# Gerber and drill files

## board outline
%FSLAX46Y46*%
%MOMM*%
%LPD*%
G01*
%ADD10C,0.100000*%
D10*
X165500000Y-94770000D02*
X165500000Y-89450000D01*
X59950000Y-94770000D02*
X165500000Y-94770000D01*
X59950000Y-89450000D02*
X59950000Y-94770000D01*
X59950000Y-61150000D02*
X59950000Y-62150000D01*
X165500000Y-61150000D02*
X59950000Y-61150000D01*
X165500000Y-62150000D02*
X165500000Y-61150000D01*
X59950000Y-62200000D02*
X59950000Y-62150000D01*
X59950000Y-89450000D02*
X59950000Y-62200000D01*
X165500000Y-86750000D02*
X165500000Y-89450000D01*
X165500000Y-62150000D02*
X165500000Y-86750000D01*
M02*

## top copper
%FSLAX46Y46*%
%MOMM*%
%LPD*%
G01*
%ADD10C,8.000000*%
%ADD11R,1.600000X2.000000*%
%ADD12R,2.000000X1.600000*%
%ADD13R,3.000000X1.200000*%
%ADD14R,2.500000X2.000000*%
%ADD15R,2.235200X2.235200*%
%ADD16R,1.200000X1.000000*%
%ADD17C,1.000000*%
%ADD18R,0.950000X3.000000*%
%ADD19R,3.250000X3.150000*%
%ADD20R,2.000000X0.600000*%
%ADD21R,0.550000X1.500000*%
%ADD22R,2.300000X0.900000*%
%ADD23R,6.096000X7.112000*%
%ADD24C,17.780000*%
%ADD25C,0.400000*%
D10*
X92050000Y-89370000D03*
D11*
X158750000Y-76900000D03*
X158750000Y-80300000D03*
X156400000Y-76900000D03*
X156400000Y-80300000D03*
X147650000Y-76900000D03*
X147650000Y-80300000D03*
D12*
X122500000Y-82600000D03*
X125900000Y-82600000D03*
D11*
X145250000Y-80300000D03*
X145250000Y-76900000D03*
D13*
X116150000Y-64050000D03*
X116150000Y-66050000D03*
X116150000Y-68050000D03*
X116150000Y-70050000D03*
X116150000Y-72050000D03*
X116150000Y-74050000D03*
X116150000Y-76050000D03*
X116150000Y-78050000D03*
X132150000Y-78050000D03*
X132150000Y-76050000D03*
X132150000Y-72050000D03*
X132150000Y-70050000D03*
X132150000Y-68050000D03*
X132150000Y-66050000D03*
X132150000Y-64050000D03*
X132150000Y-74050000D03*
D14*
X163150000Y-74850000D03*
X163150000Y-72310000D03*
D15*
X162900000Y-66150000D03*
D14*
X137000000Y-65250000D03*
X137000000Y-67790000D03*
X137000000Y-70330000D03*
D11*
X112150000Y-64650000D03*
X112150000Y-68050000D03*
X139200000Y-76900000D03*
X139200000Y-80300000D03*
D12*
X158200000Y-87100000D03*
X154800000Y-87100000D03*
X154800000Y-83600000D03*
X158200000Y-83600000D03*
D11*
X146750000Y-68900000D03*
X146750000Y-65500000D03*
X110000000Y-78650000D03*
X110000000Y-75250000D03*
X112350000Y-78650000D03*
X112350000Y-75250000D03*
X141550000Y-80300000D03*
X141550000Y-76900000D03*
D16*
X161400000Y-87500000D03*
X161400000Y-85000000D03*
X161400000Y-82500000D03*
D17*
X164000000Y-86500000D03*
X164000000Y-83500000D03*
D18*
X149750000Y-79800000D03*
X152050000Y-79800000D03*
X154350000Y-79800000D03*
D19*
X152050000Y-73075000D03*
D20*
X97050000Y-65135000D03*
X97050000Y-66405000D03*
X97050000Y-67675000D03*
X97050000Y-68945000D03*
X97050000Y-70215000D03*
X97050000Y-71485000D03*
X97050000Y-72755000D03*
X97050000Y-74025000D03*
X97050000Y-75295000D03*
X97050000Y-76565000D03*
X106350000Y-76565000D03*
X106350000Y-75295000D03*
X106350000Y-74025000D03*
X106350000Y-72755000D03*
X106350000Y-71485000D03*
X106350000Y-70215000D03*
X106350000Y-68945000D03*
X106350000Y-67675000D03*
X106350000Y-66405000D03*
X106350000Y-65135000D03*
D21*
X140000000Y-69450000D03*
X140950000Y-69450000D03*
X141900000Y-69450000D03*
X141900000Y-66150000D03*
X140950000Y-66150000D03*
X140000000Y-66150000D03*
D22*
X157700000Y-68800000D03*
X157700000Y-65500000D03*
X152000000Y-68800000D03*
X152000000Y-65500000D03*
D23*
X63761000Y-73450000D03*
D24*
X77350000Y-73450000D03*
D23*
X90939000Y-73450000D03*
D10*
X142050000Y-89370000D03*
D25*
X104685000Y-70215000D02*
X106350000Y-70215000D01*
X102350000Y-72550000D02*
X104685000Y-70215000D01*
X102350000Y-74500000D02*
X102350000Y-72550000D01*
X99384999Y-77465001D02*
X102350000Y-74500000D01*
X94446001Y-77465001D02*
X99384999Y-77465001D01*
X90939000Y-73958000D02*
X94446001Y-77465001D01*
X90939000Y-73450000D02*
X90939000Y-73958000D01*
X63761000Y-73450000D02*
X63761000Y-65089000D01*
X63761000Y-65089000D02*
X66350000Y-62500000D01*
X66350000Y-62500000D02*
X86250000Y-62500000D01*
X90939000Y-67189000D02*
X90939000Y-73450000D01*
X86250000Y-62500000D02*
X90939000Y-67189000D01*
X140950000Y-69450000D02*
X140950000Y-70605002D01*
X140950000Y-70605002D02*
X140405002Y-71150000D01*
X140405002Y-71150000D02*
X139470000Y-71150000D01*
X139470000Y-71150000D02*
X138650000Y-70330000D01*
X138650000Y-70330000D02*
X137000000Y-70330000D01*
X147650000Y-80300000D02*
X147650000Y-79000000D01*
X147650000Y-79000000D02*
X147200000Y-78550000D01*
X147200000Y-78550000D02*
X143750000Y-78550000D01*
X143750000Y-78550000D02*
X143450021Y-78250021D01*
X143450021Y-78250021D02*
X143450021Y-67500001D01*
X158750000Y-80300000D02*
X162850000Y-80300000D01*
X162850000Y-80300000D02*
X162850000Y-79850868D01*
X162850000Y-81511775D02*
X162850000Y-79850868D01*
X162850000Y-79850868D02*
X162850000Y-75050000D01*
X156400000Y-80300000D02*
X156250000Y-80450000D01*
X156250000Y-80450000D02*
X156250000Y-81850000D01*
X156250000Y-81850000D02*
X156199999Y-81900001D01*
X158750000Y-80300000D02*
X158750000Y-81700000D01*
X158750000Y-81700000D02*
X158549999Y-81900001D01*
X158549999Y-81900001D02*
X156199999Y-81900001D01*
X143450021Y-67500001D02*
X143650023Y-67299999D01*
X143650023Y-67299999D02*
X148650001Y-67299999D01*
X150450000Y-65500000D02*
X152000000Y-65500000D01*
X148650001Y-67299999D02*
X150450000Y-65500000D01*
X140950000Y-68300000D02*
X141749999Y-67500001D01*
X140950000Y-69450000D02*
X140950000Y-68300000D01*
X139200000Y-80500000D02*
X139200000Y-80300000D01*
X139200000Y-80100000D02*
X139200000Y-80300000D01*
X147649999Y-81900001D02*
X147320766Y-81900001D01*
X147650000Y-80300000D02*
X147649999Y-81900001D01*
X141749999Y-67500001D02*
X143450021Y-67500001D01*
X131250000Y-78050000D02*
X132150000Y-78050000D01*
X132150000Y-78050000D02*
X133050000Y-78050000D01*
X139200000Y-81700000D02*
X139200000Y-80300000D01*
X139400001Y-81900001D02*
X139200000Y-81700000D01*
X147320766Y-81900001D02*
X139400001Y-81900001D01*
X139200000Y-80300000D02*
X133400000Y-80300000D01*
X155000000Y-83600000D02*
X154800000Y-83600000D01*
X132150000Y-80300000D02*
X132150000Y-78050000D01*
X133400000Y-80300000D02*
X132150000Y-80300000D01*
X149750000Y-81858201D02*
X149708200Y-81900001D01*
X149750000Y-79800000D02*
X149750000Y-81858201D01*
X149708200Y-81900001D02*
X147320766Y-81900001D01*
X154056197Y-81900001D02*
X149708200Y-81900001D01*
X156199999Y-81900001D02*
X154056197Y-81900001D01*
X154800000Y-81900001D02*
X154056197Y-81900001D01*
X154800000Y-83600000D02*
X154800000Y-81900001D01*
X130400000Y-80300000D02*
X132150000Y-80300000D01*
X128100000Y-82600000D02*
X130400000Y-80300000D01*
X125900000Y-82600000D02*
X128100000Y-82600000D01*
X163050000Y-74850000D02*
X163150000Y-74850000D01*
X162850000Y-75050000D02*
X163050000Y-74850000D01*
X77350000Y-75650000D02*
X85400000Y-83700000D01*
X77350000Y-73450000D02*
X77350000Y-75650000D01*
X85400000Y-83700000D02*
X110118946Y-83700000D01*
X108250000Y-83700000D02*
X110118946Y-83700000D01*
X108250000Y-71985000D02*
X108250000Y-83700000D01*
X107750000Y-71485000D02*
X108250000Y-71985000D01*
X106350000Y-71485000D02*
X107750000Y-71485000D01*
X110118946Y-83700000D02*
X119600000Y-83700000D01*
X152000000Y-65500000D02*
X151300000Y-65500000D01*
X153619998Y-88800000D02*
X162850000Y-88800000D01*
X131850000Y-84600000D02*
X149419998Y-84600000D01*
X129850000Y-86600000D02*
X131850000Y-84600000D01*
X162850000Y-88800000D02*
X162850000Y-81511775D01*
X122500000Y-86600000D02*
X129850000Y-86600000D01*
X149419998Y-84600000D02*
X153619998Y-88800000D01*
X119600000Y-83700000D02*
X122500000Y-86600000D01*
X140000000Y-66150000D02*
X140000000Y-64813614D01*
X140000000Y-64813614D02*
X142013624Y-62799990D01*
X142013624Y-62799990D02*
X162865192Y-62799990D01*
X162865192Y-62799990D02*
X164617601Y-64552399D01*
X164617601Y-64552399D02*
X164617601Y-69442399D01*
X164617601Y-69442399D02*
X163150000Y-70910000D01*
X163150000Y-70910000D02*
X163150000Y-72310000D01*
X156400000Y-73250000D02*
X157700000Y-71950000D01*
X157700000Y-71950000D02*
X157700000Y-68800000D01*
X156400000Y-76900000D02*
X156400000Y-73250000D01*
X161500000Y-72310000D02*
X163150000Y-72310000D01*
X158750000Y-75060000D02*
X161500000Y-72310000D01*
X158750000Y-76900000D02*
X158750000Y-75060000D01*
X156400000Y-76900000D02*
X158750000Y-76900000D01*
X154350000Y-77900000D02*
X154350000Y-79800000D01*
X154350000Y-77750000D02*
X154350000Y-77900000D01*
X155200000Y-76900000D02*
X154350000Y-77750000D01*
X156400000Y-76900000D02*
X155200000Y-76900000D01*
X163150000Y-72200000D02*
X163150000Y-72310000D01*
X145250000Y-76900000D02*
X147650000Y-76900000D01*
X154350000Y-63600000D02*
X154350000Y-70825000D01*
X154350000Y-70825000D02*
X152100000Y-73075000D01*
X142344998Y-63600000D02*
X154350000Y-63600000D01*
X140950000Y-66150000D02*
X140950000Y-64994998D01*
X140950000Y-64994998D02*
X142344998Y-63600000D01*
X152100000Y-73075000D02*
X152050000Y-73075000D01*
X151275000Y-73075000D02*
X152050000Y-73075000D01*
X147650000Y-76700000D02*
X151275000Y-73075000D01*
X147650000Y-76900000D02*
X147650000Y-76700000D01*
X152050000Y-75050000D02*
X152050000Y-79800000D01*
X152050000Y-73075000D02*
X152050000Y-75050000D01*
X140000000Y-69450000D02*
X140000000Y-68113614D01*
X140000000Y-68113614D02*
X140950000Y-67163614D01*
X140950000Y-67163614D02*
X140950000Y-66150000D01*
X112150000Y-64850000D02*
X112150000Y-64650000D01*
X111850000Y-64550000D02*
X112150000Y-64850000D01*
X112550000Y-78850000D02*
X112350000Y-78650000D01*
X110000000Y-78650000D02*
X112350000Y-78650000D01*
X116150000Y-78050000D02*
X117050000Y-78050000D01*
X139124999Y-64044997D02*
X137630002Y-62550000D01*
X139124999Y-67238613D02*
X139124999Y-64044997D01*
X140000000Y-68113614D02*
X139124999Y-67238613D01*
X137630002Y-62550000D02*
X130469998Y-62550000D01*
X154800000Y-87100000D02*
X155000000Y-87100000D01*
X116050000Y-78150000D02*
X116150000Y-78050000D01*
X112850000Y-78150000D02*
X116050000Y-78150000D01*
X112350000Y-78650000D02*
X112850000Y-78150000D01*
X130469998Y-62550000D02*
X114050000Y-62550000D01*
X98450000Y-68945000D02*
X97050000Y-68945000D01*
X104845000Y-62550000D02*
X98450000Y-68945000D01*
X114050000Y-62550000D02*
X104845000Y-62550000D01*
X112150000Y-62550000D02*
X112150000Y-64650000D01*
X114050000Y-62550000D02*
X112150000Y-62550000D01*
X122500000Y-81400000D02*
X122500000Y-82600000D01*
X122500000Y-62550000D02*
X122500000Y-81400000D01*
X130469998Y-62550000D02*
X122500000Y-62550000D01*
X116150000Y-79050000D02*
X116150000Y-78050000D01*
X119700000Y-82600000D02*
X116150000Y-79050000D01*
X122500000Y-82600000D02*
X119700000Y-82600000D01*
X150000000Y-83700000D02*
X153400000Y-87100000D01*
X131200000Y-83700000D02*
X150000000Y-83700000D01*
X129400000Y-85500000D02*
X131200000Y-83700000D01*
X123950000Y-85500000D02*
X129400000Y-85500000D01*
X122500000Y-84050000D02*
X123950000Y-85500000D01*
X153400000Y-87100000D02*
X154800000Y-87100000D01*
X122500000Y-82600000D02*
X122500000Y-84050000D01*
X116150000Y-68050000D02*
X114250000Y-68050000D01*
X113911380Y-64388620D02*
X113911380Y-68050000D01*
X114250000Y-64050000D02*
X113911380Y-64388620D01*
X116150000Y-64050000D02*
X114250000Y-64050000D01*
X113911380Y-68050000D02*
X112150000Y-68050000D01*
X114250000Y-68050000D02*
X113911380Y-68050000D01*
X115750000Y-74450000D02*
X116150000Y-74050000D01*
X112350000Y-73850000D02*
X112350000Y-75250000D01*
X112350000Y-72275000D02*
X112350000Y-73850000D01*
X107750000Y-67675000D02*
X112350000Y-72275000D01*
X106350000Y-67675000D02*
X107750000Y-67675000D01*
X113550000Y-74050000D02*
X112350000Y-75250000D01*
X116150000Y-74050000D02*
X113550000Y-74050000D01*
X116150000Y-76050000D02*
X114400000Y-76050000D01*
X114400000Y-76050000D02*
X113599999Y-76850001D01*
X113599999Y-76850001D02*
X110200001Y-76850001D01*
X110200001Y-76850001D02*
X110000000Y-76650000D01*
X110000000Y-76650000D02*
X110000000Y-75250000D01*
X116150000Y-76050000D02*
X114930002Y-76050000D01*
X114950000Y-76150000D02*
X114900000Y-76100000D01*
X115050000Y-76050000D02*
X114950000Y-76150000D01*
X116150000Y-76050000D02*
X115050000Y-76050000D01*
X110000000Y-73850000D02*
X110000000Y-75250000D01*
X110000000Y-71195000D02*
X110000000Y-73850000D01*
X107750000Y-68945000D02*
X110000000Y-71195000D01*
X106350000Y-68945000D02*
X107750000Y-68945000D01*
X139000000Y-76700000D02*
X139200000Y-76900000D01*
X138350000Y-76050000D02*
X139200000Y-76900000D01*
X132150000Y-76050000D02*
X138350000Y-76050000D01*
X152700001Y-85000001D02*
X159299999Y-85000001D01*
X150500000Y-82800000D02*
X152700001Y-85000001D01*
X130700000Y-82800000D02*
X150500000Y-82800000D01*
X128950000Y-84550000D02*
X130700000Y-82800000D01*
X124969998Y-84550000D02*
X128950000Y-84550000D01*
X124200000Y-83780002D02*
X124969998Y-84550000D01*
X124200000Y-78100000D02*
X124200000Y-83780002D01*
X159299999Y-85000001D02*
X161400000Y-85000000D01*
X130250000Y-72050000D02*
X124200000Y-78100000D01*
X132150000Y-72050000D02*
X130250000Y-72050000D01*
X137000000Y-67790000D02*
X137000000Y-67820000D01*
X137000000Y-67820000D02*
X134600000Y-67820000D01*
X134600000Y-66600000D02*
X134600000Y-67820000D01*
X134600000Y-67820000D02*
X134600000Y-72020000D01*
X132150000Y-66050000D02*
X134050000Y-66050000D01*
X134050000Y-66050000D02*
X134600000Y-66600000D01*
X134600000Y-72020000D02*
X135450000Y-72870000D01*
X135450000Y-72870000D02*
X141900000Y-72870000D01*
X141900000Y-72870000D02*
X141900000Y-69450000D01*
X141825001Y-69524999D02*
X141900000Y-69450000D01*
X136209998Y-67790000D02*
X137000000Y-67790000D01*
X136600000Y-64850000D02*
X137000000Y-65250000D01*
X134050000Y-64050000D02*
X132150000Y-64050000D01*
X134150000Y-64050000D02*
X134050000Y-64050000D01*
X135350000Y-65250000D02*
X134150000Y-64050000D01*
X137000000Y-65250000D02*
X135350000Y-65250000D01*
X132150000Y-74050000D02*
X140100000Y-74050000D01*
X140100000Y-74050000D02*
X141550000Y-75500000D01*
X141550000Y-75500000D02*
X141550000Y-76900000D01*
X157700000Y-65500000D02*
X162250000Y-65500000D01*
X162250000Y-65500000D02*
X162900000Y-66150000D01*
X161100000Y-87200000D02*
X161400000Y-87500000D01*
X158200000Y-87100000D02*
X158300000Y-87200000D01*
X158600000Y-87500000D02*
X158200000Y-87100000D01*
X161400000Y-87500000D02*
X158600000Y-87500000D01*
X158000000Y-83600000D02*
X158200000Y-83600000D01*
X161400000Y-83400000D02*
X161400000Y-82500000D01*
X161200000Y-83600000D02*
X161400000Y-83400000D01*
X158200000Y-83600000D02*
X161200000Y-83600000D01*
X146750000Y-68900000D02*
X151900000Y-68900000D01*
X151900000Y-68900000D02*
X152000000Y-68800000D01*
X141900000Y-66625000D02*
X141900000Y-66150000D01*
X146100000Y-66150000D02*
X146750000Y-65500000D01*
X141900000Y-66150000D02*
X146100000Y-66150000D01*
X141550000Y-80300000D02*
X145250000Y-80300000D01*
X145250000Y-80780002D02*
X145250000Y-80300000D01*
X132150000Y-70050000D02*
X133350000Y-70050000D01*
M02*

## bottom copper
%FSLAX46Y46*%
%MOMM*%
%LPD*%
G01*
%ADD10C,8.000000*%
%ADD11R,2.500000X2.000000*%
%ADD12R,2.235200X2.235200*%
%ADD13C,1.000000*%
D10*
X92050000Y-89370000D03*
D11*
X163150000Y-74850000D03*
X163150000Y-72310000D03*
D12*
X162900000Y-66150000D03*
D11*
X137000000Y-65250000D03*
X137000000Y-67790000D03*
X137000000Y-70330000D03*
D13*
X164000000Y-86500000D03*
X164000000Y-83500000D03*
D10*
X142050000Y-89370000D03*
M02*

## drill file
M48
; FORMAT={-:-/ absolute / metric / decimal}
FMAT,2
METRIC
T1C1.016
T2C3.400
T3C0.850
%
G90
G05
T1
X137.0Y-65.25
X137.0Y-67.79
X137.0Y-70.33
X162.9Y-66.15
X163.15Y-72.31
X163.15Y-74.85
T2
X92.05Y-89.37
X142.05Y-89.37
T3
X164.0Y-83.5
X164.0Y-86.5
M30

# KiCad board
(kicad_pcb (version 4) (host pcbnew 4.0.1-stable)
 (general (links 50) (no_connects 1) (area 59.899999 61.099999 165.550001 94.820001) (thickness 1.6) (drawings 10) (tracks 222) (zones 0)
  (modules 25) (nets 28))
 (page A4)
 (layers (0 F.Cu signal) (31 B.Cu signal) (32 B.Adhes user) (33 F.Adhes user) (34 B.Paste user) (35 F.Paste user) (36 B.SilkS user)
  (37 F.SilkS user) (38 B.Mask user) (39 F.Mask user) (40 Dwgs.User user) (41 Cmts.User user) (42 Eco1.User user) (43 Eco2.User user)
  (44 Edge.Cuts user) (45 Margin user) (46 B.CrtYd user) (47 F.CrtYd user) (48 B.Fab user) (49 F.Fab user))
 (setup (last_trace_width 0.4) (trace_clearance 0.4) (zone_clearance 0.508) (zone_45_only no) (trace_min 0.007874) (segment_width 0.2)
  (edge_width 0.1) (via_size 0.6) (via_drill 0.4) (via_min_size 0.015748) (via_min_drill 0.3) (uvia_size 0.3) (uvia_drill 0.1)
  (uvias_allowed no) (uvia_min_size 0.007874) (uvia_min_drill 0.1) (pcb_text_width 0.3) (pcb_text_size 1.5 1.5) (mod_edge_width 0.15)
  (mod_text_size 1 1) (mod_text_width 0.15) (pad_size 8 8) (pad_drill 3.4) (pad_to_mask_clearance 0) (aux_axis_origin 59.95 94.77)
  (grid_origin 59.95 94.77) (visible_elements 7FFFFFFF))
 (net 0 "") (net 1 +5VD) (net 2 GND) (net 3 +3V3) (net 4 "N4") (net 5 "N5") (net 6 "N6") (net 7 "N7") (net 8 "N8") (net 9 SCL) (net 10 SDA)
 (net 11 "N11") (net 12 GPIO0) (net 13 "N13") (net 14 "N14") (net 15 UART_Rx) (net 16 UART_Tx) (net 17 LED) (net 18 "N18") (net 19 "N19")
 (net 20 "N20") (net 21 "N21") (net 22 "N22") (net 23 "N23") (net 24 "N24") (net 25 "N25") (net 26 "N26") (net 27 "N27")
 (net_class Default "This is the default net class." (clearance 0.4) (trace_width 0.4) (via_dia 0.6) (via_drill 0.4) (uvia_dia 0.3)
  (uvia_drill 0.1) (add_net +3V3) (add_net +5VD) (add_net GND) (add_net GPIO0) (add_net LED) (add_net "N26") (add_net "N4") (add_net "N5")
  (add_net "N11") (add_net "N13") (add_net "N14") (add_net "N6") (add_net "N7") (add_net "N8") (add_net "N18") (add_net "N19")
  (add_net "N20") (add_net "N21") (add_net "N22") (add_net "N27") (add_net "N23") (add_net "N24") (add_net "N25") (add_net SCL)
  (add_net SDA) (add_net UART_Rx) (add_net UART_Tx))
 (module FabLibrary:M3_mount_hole (layer F.Cu) (at 92.05 89.37)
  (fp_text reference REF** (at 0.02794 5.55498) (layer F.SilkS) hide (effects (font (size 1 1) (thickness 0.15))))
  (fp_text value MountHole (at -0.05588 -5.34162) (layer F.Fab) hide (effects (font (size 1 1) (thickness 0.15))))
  (pad 1 thru_hole circle (at 0 0) (size 8 8) (drill 3.4) (layers *.Cu *.Mask F.SilkS)))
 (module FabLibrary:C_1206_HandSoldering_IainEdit (layer F.Cu) (at 158.75 78.6 270)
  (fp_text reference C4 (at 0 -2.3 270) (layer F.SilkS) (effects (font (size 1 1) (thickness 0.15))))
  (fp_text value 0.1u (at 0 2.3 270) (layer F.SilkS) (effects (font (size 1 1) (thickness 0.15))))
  (pad 1 smd rect (at -1.7 0 270) (size 2 1.6) (layers F.Cu F.Paste F.Mask) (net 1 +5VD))
  (pad 2 smd rect (at 1.7 0 270) (size 2 1.6) (layers F.Cu F.Paste F.Mask) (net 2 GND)))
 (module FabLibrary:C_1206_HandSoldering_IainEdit (layer F.Cu) (at 156.4 78.6 270)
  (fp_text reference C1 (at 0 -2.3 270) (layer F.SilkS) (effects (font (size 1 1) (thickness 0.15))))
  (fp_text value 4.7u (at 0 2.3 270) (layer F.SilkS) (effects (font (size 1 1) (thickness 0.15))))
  (pad 1 smd rect (at -1.7 0 270) (size 2 1.6) (layers F.Cu F.Paste F.Mask) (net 1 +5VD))
  (pad 2 smd rect (at 1.7 0 270) (size 2 1.6) (layers F.Cu F.Paste F.Mask) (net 2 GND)))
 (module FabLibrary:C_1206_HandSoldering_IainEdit (layer F.Cu) (at 147.65 78.6 270)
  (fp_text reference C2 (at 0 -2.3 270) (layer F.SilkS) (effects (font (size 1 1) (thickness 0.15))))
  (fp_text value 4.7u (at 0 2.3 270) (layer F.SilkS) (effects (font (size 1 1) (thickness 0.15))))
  (pad 1 smd rect (at -1.7 0 270) (size 2 1.6) (layers F.Cu F.Paste F.Mask) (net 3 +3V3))
  (pad 2 smd rect (at 1.7 0 270) (size 2 1.6) (layers F.Cu F.Paste F.Mask) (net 2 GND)))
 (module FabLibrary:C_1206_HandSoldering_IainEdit (layer F.Cu) (at 124.2 82.6)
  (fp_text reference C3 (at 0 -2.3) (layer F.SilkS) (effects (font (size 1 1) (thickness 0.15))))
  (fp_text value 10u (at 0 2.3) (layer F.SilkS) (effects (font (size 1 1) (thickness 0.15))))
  (pad 1 smd rect (at -1.7 0) (size 2 1.6) (layers F.Cu F.Paste F.Mask) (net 3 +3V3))
  (pad 2 smd rect (at 1.7 0) (size 2 1.6) (layers F.Cu F.Paste F.Mask) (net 2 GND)))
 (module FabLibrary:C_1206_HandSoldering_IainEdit (layer F.Cu) (at 145.25 78.6 90)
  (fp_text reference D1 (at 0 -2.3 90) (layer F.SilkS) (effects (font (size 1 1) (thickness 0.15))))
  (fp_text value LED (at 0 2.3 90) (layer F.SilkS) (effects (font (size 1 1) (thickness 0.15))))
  (pad 1 smd rect (at -1.7 0 90) (size 2 1.6) (layers F.Cu F.Paste F.Mask) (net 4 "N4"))
  (pad 2 smd rect (at 1.7 0 90) (size 2 1.6) (layers F.Cu F.Paste F.Mask) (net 3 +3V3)))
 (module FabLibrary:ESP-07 (layer F.Cu) (at 124.15 70.05 270)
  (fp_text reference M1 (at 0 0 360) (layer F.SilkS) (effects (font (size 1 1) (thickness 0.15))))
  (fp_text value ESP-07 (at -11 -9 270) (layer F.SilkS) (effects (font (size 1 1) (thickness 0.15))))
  (pad 1 smd rect (at -6 8 270) (size 1.2 3) (layers F.Cu F.Paste F.Mask) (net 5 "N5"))
  (pad 2 smd rect (at -4 8 270) (size 1.2 3) (layers F.Cu F.Paste F.Mask) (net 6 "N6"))
  (pad 3 smd rect (at -2 8 270) (size 1.2 3) (layers F.Cu F.Paste F.Mask) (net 5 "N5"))
  (pad 4 smd rect (at 0 8 270) (size 1.2 3) (layers F.Cu F.Paste F.Mask) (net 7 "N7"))
  (pad 5 smd rect (at 2 8 270) (size 1.2 3) (layers F.Cu F.Paste F.Mask) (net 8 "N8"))
  (pad 6 smd rect (at 4 8 270) (size 1.2 3) (layers F.Cu F.Paste F.Mask) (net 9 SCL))
  (pad 7 smd rect (at 6 8 270) (size 1.2 3) (layers F.Cu F.Paste F.Mask) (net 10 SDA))
  (pad 8 smd rect (at 8 8 270) (size 1.2 3) (layers F.Cu F.Paste F.Mask) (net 3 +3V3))
  (pad 9 smd rect (at 8 -8 270) (size 1.2 3) (layers F.Cu F.Paste F.Mask) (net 2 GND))
  (pad 10 smd rect (at 6 -8 270) (size 1.2 3) (layers F.Cu F.Paste F.Mask) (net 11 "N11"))
  (pad 12 smd rect (at 2 -8 270) (size 1.2 3) (layers F.Cu F.Paste F.Mask) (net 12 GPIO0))
  (pad 13 smd rect (at 0 -8 270) (size 1.2 3) (layers F.Cu F.Paste F.Mask) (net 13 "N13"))
  (pad 14 smd rect (at -2 -8 270) (size 1.2 3) (layers F.Cu F.Paste F.Mask) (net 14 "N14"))
  (pad 15 smd rect (at -4 -8 270) (size 1.2 3) (layers F.Cu F.Paste F.Mask) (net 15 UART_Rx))
  (pad 16 smd rect (at -6 -8 270) (size 1.2 3) (layers F.Cu F.Paste F.Mask) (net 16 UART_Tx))
  (pad 11 smd rect (at 4 -8 270) (size 1.2 3) (layers F.Cu F.Paste F.Mask) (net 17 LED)))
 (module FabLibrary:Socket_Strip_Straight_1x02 (layer F.Cu) (at 163.15 74.85 90)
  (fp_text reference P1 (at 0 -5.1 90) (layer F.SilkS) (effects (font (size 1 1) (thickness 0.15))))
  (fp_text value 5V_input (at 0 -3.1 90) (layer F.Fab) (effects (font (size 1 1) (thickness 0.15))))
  (pad 1 thru_hole rect (at 0 0 90) (size 2 2.5) (drill 1.016) (layers *.Mask F.Cu F.SilkS) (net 2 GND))
  (pad 2 thru_hole rect (at 2.54 0 90) (size 2 2.5) (drill 1.016) (layers *.Mask F.Cu F.SilkS) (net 1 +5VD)))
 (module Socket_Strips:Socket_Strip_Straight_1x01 (layer F.Cu) (at 162.9 66.15)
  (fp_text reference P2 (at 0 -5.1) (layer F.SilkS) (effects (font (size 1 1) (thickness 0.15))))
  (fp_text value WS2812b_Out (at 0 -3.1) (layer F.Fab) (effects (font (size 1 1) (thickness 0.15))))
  (pad 1 thru_hole rect (at 0 0) (size 2.2352 2.2352) (drill 1.016) (layers *.Cu *.Mask F.SilkS) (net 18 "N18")))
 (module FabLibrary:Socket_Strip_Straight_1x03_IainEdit (layer F.Cu) (at 137 65.25 270)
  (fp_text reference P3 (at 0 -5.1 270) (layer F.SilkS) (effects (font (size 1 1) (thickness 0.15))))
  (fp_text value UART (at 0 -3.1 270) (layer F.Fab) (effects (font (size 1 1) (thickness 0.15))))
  (pad 1 thru_hole rect (at 0 0 270) (size 2 2.5) (drill 1.016) (layers *.Mask F.Cu F.SilkS) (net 16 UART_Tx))
  (pad 2 thru_hole rect (at 2.54 0 270) (size 2 2.5) (drill 1.016) (layers *.Mask F.Cu F.SilkS) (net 15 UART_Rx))
  (pad 3 thru_hole rect (at 5.08 0 270) (size 2 2.5) (drill 1.016) (layers *.Mask F.Cu F.SilkS) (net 2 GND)))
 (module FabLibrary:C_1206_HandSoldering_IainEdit (layer F.Cu) (at 112.15 66.35 270)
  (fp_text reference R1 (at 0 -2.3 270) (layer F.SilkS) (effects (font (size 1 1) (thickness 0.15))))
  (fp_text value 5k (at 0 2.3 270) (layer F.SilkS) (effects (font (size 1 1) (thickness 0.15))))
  (pad 1 smd rect (at -1.7 0 270) (size 2 1.6) (layers F.Cu F.Paste F.Mask) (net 3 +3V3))
  (pad 2 smd rect (at 1.7 0 270) (size 2 1.6) (layers F.Cu F.Paste F.Mask) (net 5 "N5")))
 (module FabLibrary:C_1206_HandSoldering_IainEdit (layer F.Cu) (at 139.2 78.6 270)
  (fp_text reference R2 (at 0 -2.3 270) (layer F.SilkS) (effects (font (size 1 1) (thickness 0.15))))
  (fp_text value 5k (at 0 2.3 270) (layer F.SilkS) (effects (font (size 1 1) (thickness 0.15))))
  (pad 1 smd rect (at -1.7 0 270) (size 2 1.6) (layers F.Cu F.Paste F.Mask) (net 11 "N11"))
  (pad 2 smd rect (at 1.7 0 270) (size 2 1.6) (layers F.Cu F.Paste F.Mask) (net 2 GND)))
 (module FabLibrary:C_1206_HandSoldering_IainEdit (layer F.Cu) (at 156.5 87.1 180)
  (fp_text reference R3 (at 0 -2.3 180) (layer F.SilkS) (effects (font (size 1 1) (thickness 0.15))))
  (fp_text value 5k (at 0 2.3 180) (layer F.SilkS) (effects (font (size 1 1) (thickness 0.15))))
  (pad 1 smd rect (at -1.7 0 180) (size 2 1.6) (layers F.Cu F.Paste F.Mask) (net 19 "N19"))
  (pad 2 smd rect (at 1.7 0 180) (size 2 1.6) (layers F.Cu F.Paste F.Mask) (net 3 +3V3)))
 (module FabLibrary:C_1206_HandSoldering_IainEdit (layer F.Cu) (at 156.5 83.6)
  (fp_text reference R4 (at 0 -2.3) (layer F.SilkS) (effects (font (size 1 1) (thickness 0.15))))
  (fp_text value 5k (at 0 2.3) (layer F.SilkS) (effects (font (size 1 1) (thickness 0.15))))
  (pad 1 smd rect (at -1.7 0) (size 2 1.6) (layers F.Cu F.Paste F.Mask) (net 2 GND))
  (pad 2 smd rect (at 1.7 0) (size 2 1.6) (layers F.Cu F.Paste F.Mask) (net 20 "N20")))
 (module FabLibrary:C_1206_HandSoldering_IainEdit (layer F.Cu) (at 146.75 67.2 90)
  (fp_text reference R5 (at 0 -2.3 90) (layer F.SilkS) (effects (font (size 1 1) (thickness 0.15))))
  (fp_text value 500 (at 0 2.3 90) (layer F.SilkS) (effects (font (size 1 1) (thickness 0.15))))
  (pad 1 smd rect (at -1.7 0 90) (size 2 1.6) (layers F.Cu F.Paste F.Mask) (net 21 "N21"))
  (pad 2 smd rect (at 1.7 0 90) (size 2 1.6) (layers F.Cu F.Paste F.Mask) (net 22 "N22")))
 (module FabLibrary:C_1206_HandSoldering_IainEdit (layer F.Cu) (at 110 76.95 90)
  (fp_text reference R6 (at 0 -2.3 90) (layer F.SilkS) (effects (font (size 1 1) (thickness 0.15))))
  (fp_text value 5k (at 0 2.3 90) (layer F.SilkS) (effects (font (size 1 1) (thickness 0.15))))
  (pad 1 smd rect (at -1.7 0 90) (size 2 1.6) (layers F.Cu F.Paste F.Mask) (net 3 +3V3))
  (pad 2 smd rect (at 1.7 0 90) (size 2 1.6) (layers F.Cu F.Paste F.Mask) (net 10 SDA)))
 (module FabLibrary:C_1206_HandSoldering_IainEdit (layer F.Cu) (at 112.35 76.95 90)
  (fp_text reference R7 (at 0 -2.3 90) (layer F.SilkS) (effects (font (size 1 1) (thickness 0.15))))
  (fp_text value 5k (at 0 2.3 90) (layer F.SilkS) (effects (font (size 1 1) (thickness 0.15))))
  (pad 1 smd rect (at -1.7 0 90) (size 2 1.6) (layers F.Cu F.Paste F.Mask) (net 3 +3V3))
  (pad 2 smd rect (at 1.7 0 90) (size 2 1.6) (layers F.Cu F.Paste F.Mask) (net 9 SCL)))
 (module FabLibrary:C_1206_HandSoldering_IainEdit (layer F.Cu) (at 141.55 78.6 90)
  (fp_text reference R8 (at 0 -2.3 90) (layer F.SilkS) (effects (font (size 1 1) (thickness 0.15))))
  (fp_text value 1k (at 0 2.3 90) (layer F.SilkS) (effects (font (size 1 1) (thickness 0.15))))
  (pad 1 smd rect (at -1.7 0 90) (size 2 1.6) (layers F.Cu F.Paste F.Mask) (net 4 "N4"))
  (pad 2 smd rect (at 1.7 0 90) (size 2 1.6) (layers F.Cu F.Paste F.Mask) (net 17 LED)))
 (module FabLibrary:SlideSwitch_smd (layer F.Cu) (at 164 85 90)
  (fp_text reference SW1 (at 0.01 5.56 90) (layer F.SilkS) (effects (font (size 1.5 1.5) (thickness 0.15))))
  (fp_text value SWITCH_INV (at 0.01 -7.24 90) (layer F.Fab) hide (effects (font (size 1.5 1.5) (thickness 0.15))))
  (pad 1 smd rect (at -2.5 -2.6 90) (size 1 1.2) (layers F.Cu F.Paste F.Mask) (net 19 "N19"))
  (pad 2 smd rect (at 0 -2.6 90) (size 1 1.2) (layers F.Cu F.Paste F.Mask) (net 12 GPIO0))
  (pad 3 smd rect (at 2.5 -2.6 90) (size 1 1.2) (layers F.Cu F.Paste F.Mask) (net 20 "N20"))
  (pad "" np_thru_hole circle (at -1.5 0 90) (size 1 1) (drill 0.85) (layers *.Cu *.Mask F.SilkS))
  (pad "" np_thru_hole circle (at 1.5 0 90) (size 1 1) (drill 0.85) (layers *.Cu *.Mask F.SilkS)))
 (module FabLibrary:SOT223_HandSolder (layer F.Cu) (at 152.05 78.3)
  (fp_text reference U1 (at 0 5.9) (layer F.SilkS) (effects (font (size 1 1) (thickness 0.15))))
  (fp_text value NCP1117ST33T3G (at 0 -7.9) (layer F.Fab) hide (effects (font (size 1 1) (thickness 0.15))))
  (pad 1 smd rect (at -2.3 1.5) (size 0.95 3) (layers F.Cu F.Paste F.Mask) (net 2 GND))
  (pad 2 smd rect (at 0 1.5) (size 0.95 3) (layers F.Cu F.Paste F.Mask) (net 3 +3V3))
  (pad 3 smd rect (at 2.3 1.5) (size 0.95 3) (layers F.Cu F.Paste F.Mask) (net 1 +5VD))
  (pad 2 smd rect (at 0 -5.225) (size 3.25 3.15) (layers F.Cu F.Paste F.Mask) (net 3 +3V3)))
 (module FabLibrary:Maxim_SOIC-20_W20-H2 (layer F.Cu) (at 101.7 70.85 270)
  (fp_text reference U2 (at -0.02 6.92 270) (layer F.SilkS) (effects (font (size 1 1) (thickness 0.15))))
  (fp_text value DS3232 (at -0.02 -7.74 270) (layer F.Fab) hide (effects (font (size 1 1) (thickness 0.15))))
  (pad 1 smd rect (at -5.715 4.65 270) (size 0.6 2) (layers F.Cu F.Paste F.Mask))
  (pad 2 smd rect (at -4.445 4.65 270) (size 0.6 2) (layers F.Cu F.Paste F.Mask))
  (pad 3 smd rect (at -3.175 4.65 270) (size 0.6 2) (layers F.Cu F.Paste F.Mask) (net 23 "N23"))
  (pad 4 smd rect (at -1.905 4.65 270) (size 0.6 2) (layers F.Cu F.Paste F.Mask) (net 3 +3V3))
  (pad 5 smd rect (at -0.635 4.65 270) (size 0.6 2) (layers F.Cu F.Paste F.Mask) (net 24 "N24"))
  (pad 6 smd rect (at 0.635 4.65 270) (size 0.6 2) (layers F.Cu F.Paste F.Mask) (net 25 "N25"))
  (pad 7 smd rect (at 1.905 4.65 270) (size 0.6 2) (layers F.Cu F.Paste F.Mask))
  (pad 8 smd rect (at 3.175 4.65 270) (size 0.6 2) (layers F.Cu F.Paste F.Mask))
  (pad 9 smd rect (at 4.445 4.65 270) (size 0.6 2) (layers F.Cu F.Paste F.Mask))
  (pad 10 smd rect (at 5.715 4.65 270) (size 0.6 2) (layers F.Cu F.Paste F.Mask))
  (pad 11 smd rect (at 5.715 -4.65 270) (size 0.6 2) (layers F.Cu F.Paste F.Mask))
  (pad 12 smd rect (at 4.445 -4.65 270) (size 0.6 2) (layers F.Cu F.Paste F.Mask))
  (pad 13 smd rect (at 3.175 -4.65 270) (size 0.6 2) (layers F.Cu F.Paste F.Mask))
  (pad 14 smd rect (at 1.905 -4.65 270) (size 0.6 2) (layers F.Cu F.Paste F.Mask))
  (pad 15 smd rect (at 0.635 -4.65 270) (size 0.6 2) (layers F.Cu F.Paste F.Mask) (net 2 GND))
  (pad 16 smd rect (at -0.635 -4.65 270) (size 0.6 2) (layers F.Cu F.Paste F.Mask) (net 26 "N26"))
  (pad 17 smd rect (at -1.905 -4.65 270) (size 0.6 2) (layers F.Cu F.Paste F.Mask) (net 10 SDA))
  (pad 18 smd rect (at -3.175 -4.65 270) (size 0.6 2) (layers F.Cu F.Paste F.Mask) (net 9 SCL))
  (pad 19 smd rect (at -4.445 -4.65 270) (size 0.6 2) (layers F.Cu F.Paste F.Mask))
  (pad 20 smd rect (at -5.715 -4.65 270) (size 0.6 2) (layers F.Cu F.Paste F.Mask) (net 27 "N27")))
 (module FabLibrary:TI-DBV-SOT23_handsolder (layer F.Cu) (at 140.95 67.85)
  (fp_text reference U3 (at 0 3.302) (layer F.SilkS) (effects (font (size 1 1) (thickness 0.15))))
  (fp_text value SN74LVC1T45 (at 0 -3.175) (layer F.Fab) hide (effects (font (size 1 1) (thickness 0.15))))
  (pad 1 smd rect (at -0.95 1.6) (size 0.55 1.5) (layers F.Cu F.Paste F.Mask) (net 3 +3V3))
  (pad 2 smd rect (at 0 1.6) (size 0.55 1.5) (layers F.Cu F.Paste F.Mask) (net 2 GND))
  (pad 3 smd rect (at 0.95 1.6) (size 0.55 1.5) (layers F.Cu F.Paste F.Mask) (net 15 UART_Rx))
  (pad 4 smd rect (at 0.95 -1.7) (size 0.55 1.5) (layers F.Cu F.Paste F.Mask) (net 22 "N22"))
  (pad 5 smd rect (at 0 -1.7) (size 0.55 1.5) (layers F.Cu F.Paste F.Mask) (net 3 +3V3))
  (pad 6 smd rect (at -0.95 -1.7) (size 0.55 1.5) (layers F.Cu F.Paste F.Mask) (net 1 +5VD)))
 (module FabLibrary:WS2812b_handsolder (layer F.Cu) (at 154.85 67.15 180)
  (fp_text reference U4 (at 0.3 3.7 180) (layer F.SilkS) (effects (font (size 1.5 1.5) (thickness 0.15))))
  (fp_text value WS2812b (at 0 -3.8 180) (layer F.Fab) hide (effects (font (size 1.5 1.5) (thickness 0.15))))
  (pad 1 smd rect (at -2.85 -1.65 180) (size 2.3 0.9) (layers F.Cu F.Paste F.Mask) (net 1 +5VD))
  (pad 2 smd rect (at -2.85 1.65 180) (size 2.3 0.9) (layers F.Cu F.Paste F.Mask) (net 18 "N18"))
  (pad 4 smd rect (at 2.85 -1.65 180) (size 2.3 0.9) (layers F.Cu F.Paste F.Mask) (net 21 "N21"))
  (pad 3 smd rect (at 2.85 1.65 180) (size 2.3 0.9) (layers F.Cu F.Paste F.Mask) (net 2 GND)))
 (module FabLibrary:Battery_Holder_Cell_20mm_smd (layer F.Cu) (at 77.35 73.45 180)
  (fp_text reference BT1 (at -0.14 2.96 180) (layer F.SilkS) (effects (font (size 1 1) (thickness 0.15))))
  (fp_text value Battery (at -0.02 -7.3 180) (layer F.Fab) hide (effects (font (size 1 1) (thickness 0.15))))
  (pad 1 smd rect (at 13.589 0 180) (size 6.096 7.112) (layers F.Cu F.Paste F.Mask) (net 26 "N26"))
  (pad 2 smd circle (at 0 0 180) (size 17.78 17.78) (layers F.Cu F.Paste F.Mask) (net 2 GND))
  (pad 1 smd rect (at -13.589 0 180) (size 6.096 7.112) (layers F.Cu F.Paste F.Mask) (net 26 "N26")))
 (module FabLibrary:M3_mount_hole (layer F.Cu) (at 142.05 89.37)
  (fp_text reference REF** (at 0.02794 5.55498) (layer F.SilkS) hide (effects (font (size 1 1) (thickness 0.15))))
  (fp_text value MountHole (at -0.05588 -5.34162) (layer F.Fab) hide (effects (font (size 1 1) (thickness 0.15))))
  (pad 1 thru_hole circle (at 0 0) (size 8 8) (drill 3.4) (layers *.Cu *.Mask F.SilkS)))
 (gr_line (start 165.5 94.77) (end 165.5 89.45) (angle 90) (layer Edge.Cuts) (width 0.1))
 (gr_line (start 59.95 94.77) (end 165.5 94.77) (angle 90) (layer Edge.Cuts) (width 0.1))
 (gr_line (start 59.95 89.45) (end 59.95 94.77) (angle 90) (layer Edge.Cuts) (width 0.1))
 (gr_line (start 59.95 61.15) (end 59.95 62.15) (angle 90) (layer Edge.Cuts) (width 0.1))
 (gr_line (start 165.5 61.15) (end 59.95 61.15) (angle 90) (layer Edge.Cuts) (width 0.1))
 (gr_line (start 165.5 62.15) (end 165.5 61.15) (angle 90) (layer Edge.Cuts) (width 0.1))
 (gr_line (start 59.95 62.2) (end 59.95 62.15) (layer Edge.Cuts) (width 0.1))
 (gr_line (start 59.95 89.45) (end 59.95 62.2) (layer Edge.Cuts) (width 0.1))
 (gr_line (start 165.5 86.75) (end 165.5 89.45) (layer Edge.Cuts) (width 0.1))
 (gr_line (start 165.5 62.15) (end 165.5 86.75) (layer Edge.Cuts) (width 0.1))
 (segment (start 104.685 70.215) (end 106.35 70.215) (width 0.4) (layer F.Cu) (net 26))
 (segment (start 102.35 72.55) (end 104.685 70.215) (width 0.4) (layer F.Cu) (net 26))
 (segment (start 102.35 74.5) (end 102.35 72.55) (width 0.4) (layer F.Cu) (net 26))
 (segment (start 99.384999 77.465001) (end 102.35 74.5) (width 0.4) (layer F.Cu) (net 26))
 (segment (start 94.446001 77.465001) (end 99.384999 77.465001) (width 0.4) (layer F.Cu) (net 26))
 (segment (start 90.939 73.958) (end 94.446001 77.465001) (width 0.4) (layer F.Cu) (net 26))
 (segment (start 90.939 73.45) (end 90.939 73.958) (width 0.4) (layer F.Cu) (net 26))
 (segment (start 63.761 73.45) (end 63.761 65.089) (width 0.4) (layer F.Cu) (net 26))
 (segment (start 63.761 65.089) (end 66.35 62.5) (width 0.4) (layer F.Cu) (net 26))
 (segment (start 66.35 62.5) (end 86.25 62.5) (width 0.4) (layer F.Cu) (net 26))
 (segment (start 90.939 67.189) (end 90.939 73.45) (width 0.4) (layer F.Cu) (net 26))
 (segment (start 86.25 62.5) (end 90.939 67.189) (width 0.4) (layer F.Cu) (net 26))
 (segment (start 140.95 69.45) (end 140.95 70.605002) (width 0.4) (layer F.Cu) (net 2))
 (segment (start 140.95 70.605002) (end 140.405002 71.15) (width 0.4) (layer F.Cu) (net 2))
 (segment (start 140.405002 71.15) (end 139.47 71.15) (width 0.4) (layer F.Cu) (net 2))
 (segment (start 139.47 71.15) (end 138.65 70.33) (width 0.4) (layer F.Cu) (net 2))
 (segment (start 138.65 70.33) (end 137 70.33) (width 0.4) (layer F.Cu) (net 2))
 (segment (start 147.65 80.3) (end 147.65 79) (width 0.4) (layer F.Cu) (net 2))
 (segment (start 147.65 79) (end 147.2 78.55) (width 0.4) (layer F.Cu) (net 2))
 (segment (start 147.2 78.55) (end 143.75 78.55) (width 0.4) (layer F.Cu) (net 2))
 (segment (start 143.75 78.55) (end 143.450021 78.250021) (width 0.4) (layer F.Cu) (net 2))
 (segment (start 143.450021 78.250021) (end 143.450021 67.500001) (width 0.4) (layer F.Cu) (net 2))
 (segment (start 158.75 80.3) (end 162.85 80.3) (width 0.4) (layer F.Cu) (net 2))
 (segment (start 162.85 80.3) (end 162.85 79.850868) (width 0.4) (layer F.Cu) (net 2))
 (segment (start 162.85 81.511775) (end 162.85 79.850868) (width 0.4) (layer F.Cu) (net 2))
 (segment (start 162.85 79.850868) (end 162.85 75.05) (width 0.4) (layer F.Cu) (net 2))
 (segment (start 156.4 80.3) (end 156.25 80.45) (width 0.4) (layer F.Cu) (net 2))
 (segment (start 156.25 80.45) (end 156.25 81.85) (width 0.4) (layer F.Cu) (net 2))
 (segment (start 156.25 81.85) (end 156.199999 81.900001) (width 0.4) (layer F.Cu) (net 2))
 (segment (start 158.75 80.3) (end 158.75 81.7) (width 0.4) (layer F.Cu) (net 2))
 (segment (start 158.75 81.7) (end 158.549999 81.900001) (width 0.4) (layer F.Cu) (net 2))
 (segment (start 158.549999 81.900001) (end 156.199999 81.900001) (width 0.4) (layer F.Cu) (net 2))
 (segment (start 143.450021 67.500001) (end 143.650023 67.299999) (width 0.4) (layer F.Cu) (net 2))
 (segment (start 143.650023 67.299999) (end 148.650001 67.299999) (width 0.4) (layer F.Cu) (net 2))
 (segment (start 150.45 65.5) (end 152 65.5) (width 0.4) (layer F.Cu) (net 2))
 (segment (start 148.650001 67.299999) (end 150.45 65.5) (width 0.4) (layer F.Cu) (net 2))
 (segment (start 140.95 68.3) (end 141.749999 67.500001) (width 0.4) (layer F.Cu) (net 2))
 (segment (start 140.95 69.45) (end 140.95 68.3) (width 0.4) (layer F.Cu) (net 2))
 (segment (start 139.2 80.5) (end 139.2 80.3) (width 0.4) (layer F.Cu) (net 2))
 (segment (start 139.2 80.1) (end 139.2 80.3) (width 0.4) (layer F.Cu) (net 2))
 (segment (start 147.649999 81.900001) (end 147.320766 81.900001) (width 0.4) (layer F.Cu) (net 2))
 (segment (start 147.65 80.3) (end 147.649999 81.900001) (width 0.4) (layer F.Cu) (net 2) (status 10))
 (segment (start 141.749999 67.500001) (end 143.450021 67.500001) (width 0.4) (layer F.Cu) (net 2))
 (segment (start 131.25 78.05) (end 132.15 78.05) (width 0.4) (layer F.Cu) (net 2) (status 30))
 (segment (start 132.15 78.05) (end 133.05 78.05) (width 0.4) (layer F.Cu) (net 2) (status 30))
 (segment (start 139.2 81.7) (end 139.2 80.3) (width 0.4) (layer F.Cu) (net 2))
 (segment (start 139.400001 81.900001) (end 139.2 81.7) (width 0.4) (layer F.Cu) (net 2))
 (segment (start 147.320766 81.900001) (end 139.400001 81.900001) (width 0.4) (layer F.Cu) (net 2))
 (segment (start 139.2 80.3) (end 133.4 80.3) (width 0.4) (layer F.Cu) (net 2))
 (segment (start 155 83.6) (end 154.8 83.6) (width 0.4) (layer F.Cu) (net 2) (status 30))
 (segment (start 132.15 80.3) (end 132.15 78.05) (width 0.4) (layer F.Cu) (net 2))
 (segment (start 133.4 80.3) (end 132.15 80.3) (width 0.4) (layer F.Cu) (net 2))
 (segment (start 149.75 81.858201) (end 149.7082 81.900001) (width 0.4) (layer F.Cu) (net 2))
 (segment (start 149.75 79.8) (end 149.75 81.858201) (width 0.4) (layer F.Cu) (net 2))
 (segment (start 149.7082 81.900001) (end 147.320766 81.900001) (width 0.4) (layer F.Cu) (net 2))
 (segment (start 154.056197 81.900001) (end 149.7082 81.900001) (width 0.4) (layer F.Cu) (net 2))
 (segment (start 156.199999 81.900001) (end 154.056197 81.900001) (width 0.4) (layer F.Cu) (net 2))
 (segment (start 154.8 81.900001) (end 154.056197 81.900001) (width 0.4) (layer F.Cu) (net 2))
 (segment (start 154.8 83.6) (end 154.8 81.900001) (width 0.4) (layer F.Cu) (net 2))
 (segment (start 130.4 80.3) (end 132.15 80.3) (width 0.4) (layer F.Cu) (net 2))
 (segment (start 128.1 82.6) (end 130.4 80.3) (width 0.4) (layer F.Cu) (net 2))
 (segment (start 125.9 82.6) (end 128.1 82.6) (width 0.4) (layer F.Cu) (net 2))
 (segment (start 163.05 74.85) (end 163.15 74.85) (width 0.4) (layer F.Cu) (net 2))
 (segment (start 162.85 75.05) (end 163.05 74.85) (width 0.4) (layer F.Cu) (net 2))
 (segment (start 77.35 75.65) (end 85.4 83.7) (width 0.4) (layer F.Cu) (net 2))
 (segment (start 77.35 73.45) (end 77.35 75.65) (width 0.4) (layer F.Cu) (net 2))
 (segment (start 85.4 83.7) (end 110.118946 83.7) (width 0.4) (layer F.Cu) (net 2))
 (segment (start 108.25 83.7) (end 110.118946 83.7) (width 0.4) (layer F.Cu) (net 2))
 (segment (start 108.25 71.985) (end 108.25 83.7) (width 0.4) (layer F.Cu) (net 2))
 (segment (start 107.75 71.485) (end 108.25 71.985) (width 0.4) (layer F.Cu) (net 2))
 (segment (start 106.35 71.485) (end 107.75 71.485) (width 0.4) (layer F.Cu) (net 2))
 (segment (start 110.118946 83.7) (end 119.6 83.7) (width 0.4) (layer F.Cu) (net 2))
 (segment (start 152 65.5) (end 151.3 65.5) (width 0.4) (layer F.Cu) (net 2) (status 30))
 (segment (start 153.619998 88.8) (end 162.85 88.8) (width 0.4) (layer F.Cu) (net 2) (status 20))
 (segment (start 131.85 84.6) (end 149.419998 84.6) (width 0.4) (layer F.Cu) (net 2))
 (segment (start 129.85 86.6) (end 131.85 84.6) (width 0.4) (layer F.Cu) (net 2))
 (segment (start 162.85 88.8) (end 162.85 81.511775) (width 0.4) (layer F.Cu) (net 2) (status 10))
 (segment (start 122.5 86.6) (end 129.85 86.6) (width 0.4) (layer F.Cu) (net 2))
 (segment (start 149.419998 84.6) (end 153.619998 88.8) (width 0.4) (layer F.Cu) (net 2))
 (segment (start 119.6 83.7) (end 122.5 86.6) (width 0.4) (layer F.Cu) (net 2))
 (segment (start 140 66.15) (end 140 64.813614) (width 0.4) (layer F.Cu) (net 1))
 (segment (start 140 64.813614) (end 142.013624 62.79999) (width 0.4) (layer F.Cu) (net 1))
 (segment (start 142.013624 62.79999) (end 162.865192 62.79999) (width 0.4) (layer F.Cu) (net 1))
 (segment (start 162.865192 62.79999) (end 164.617601 64.552399) (width 0.4) (layer F.Cu) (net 1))
 (segment (start 164.617601 64.552399) (end 164.617601 69.442399) (width 0.4) (layer F.Cu) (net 1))
 (segment (start 164.617601 69.442399) (end 163.15 70.91) (width 0.4) (layer F.Cu) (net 1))
 (segment (start 163.15 70.91) (end 163.15 72.31) (width 0.4) (layer F.Cu) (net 1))
 (segment (start 156.4 73.25) (end 157.7 71.95) (width 0.4) (layer F.Cu) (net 1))
 (segment (start 157.7 71.95) (end 157.7 68.8) (width 0.4) (layer F.Cu) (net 1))
 (segment (start 156.4 76.9) (end 156.4 73.25) (width 0.4) (layer F.Cu) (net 1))
 (segment (start 161.5 72.31) (end 163.15 72.31) (width 0.4) (layer F.Cu) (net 1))
 (segment (start 158.75 75.06) (end 161.5 72.31) (width 0.4) (layer F.Cu) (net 1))
 (segment (start 158.75 76.9) (end 158.75 75.06) (width 0.4) (layer F.Cu) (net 1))
 (segment (start 156.4 76.9) (end 158.75 76.9) (width 0.4) (layer F.Cu) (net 1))
 (segment (start 154.35 77.9) (end 154.35 79.8) (width 0.4) (layer F.Cu) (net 1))
 (segment (start 154.35 77.75) (end 154.35 77.9) (width 0.4) (layer F.Cu) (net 1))
 (segment (start 155.2 76.9) (end 154.35 77.75) (width 0.4) (layer F.Cu) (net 1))
 (segment (start 156.4 76.9) (end 155.2 76.9) (width 0.4) (layer F.Cu) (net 1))
 (segment (start 163.15 72.2) (end 163.15 72.31) (width 0.4) (layer F.Cu) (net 1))
 (segment (start 145.25 76.9) (end 147.65 76.9) (width 0.4) (layer F.Cu) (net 3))
 (segment (start 154.35 63.6) (end 154.35 70.825) (width 0.4) (layer F.Cu) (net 3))
 (segment (start 154.35 70.825) (end 152.1 73.075) (width 0.4) (layer F.Cu) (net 3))
 (segment (start 142.344998 63.6) (end 154.35 63.6) (width 0.4) (layer F.Cu) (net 3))
 (segment (start 140.95 66.15) (end 140.95 64.994998) (width 0.4) (layer F.Cu) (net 3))
 (segment (start 140.95 64.994998) (end 142.344998 63.6) (width 0.4) (layer F.Cu) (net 3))
 (segment (start 152.1 73.075) (end 152.05 73.075) (width 0.4) (layer F.Cu) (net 3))
 (segment (start 151.275 73.075) (end 152.05 73.075) (width 0.4) (layer F.Cu) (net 3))
 (segment (start 147.65 76.7) (end 151.275 73.075) (width 0.4) (layer F.Cu) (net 3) (status 10))
 (segment (start 147.65 76.9) (end 147.65 76.7) (width 0.4) (layer F.Cu) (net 3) (status 30))
 (segment (start 152.05 75.05) (end 152.05 79.8) (width 0.4) (layer F.Cu) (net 3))
 (segment (start 152.05 73.075) (end 152.05 75.05) (width 0.4) (layer F.Cu) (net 3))
 (segment (start 140 69.45) (end 140 68.113614) (width 0.4) (layer F.Cu) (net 3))
 (segment (start 140 68.113614) (end 140.95 67.163614) (width 0.4) (layer F.Cu) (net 3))
 (segment (start 140.95 67.163614) (end 140.95 66.15) (width 0.4) (layer F.Cu) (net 3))
 (segment (start 112.15 64.85) (end 112.15 64.65) (width 0.4) (layer F.Cu) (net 3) (status 30))
 (segment (start 111.85 64.55) (end 112.15 64.85) (width 0.4) (layer F.Cu) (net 3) (status 30))
 (segment (start 112.55 78.85) (end 112.35 78.65) (width 0.4) (layer F.Cu) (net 3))
 (segment (start 110 78.65) (end 112.35 78.65) (width 0.4) (layer F.Cu) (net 3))
 (segment (start 116.15 78.05) (end 117.05 78.05) (width 0.4) (layer F.Cu) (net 3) (status 30))
 (segment (start 139.124999 64.044997) (end 137.630002 62.55) (width 0.4) (layer F.Cu) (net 3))
 (segment (start 139.124999 67.238613) (end 139.124999 64.044997) (width 0.4) (layer F.Cu) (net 3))
 (segment (start 140 68.113614) (end 139.124999 67.238613) (width 0.4) (layer F.Cu) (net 3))
 (segment (start 137.630002 62.55) (end 130.469998 62.55) (width 0.4) (layer F.Cu) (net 3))
 (segment (start 154.8 87.1) (end 155 87.1) (width 0.4) (layer F.Cu) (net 3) (status 30))
 (segment (start 116.05 78.15) (end 116.15 78.05) (width 0.4) (layer F.Cu) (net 3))
 (segment (start 112.85 78.15) (end 116.05 78.15) (width 0.4) (layer F.Cu) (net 3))
 (segment (start 112.35 78.65) (end 112.85 78.15) (width 0.4) (layer F.Cu) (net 3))
 (segment (start 130.469998 62.55) (end 114.05 62.55) (width 0.4) (layer F.Cu) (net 3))
 (segment (start 98.45 68.945) (end 97.05 68.945) (width 0.4) (layer F.Cu) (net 3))
 (segment (start 104.845 62.55) (end 98.45 68.945) (width 0.4) (layer F.Cu) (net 3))
 (segment (start 114.05 62.55) (end 104.845 62.55) (width 0.4) (layer F.Cu) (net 3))
 (segment (start 112.15 62.55) (end 112.15 64.65) (width 0.4) (layer F.Cu) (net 3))
 (segment (start 114.05 62.55) (end 112.15 62.55) (width 0.4) (layer F.Cu) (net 3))
 (segment (start 122.5 81.4) (end 122.5 82.6) (width 0.4) (layer F.Cu) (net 3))
 (segment (start 122.5 62.55) (end 122.5 81.4) (width 0.4) (layer F.Cu) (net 3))
 (segment (start 130.469998 62.55) (end 122.5 62.55) (width 0.4) (layer F.Cu) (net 3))
 (segment (start 116.15 79.05) (end 116.15 78.05) (width 0.4) (layer F.Cu) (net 3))
 (segment (start 119.7 82.6) (end 116.15 79.05) (width 0.4) (layer F.Cu) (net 3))
 (segment (start 122.5 82.6) (end 119.7 82.6) (width 0.4) (layer F.Cu) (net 3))
 (segment (start 150 83.7) (end 153.4 87.1) (width 0.4) (layer F.Cu) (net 3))
 (segment (start 131.2 83.7) (end 150 83.7) (width 0.4) (layer F.Cu) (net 3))
 (segment (start 129.4 85.5) (end 131.2 83.7) (width 0.4) (layer F.Cu) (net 3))
 (segment (start 123.95 85.5) (end 129.4 85.5) (width 0.4) (layer F.Cu) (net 3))
 (segment (start 122.5 84.05) (end 123.95 85.5) (width 0.4) (layer F.Cu) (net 3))
 (segment (start 153.4 87.1) (end 154.8 87.1) (width 0.4) (layer F.Cu) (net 3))
 (segment (start 122.5 82.6) (end 122.5 84.05) (width 0.4) (layer F.Cu) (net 3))
 (segment (start 116.15 68.05) (end 114.25 68.05) (width 0.4) (layer F.Cu) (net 5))
 (segment (start 113.91138 64.38862) (end 113.91138 68.05) (width 0.4) (layer F.Cu) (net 5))
 (segment (start 114.25 64.05) (end 113.91138 64.38862) (width 0.4) (layer F.Cu) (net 5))
 (segment (start 116.15 64.05) (end 114.25 64.05) (width 0.4) (layer F.Cu) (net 5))
 (segment (start 113.91138 68.05) (end 112.15 68.05) (width 0.4) (layer F.Cu) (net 5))
 (segment (start 114.25 68.05) (end 113.91138 68.05) (width 0.4) (layer F.Cu) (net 5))
 (segment (start 115.75 74.45) (end 116.15 74.05) (width 0.4) (layer F.Cu) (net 9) (status 30))
 (segment (start 112.35 73.85) (end 112.35 75.25) (width 0.4) (layer F.Cu) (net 9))
 (segment (start 112.35 72.275) (end 112.35 73.85) (width 0.4) (layer F.Cu) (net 9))
 (segment (start 107.75 67.675) (end 112.35 72.275) (width 0.4) (layer F.Cu) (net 9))
 (segment (start 106.35 67.675) (end 107.75 67.675) (width 0.4) (layer F.Cu) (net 9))
 (segment (start 113.55 74.05) (end 112.35 75.25) (width 0.4) (layer F.Cu) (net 9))
 (segment (start 116.15 74.05) (end 113.55 74.05) (width 0.4) (layer F.Cu) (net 9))
 (segment (start 116.15 76.05) (end 114.4 76.05) (width 0.4) (layer F.Cu) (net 10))
 (segment (start 114.4 76.05) (end 113.599999 76.850001) (width 0.4) (layer F.Cu) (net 10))
 (segment (start 113.599999 76.850001) (end 110.200001 76.850001) (width 0.4) (layer F.Cu) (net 10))
 (segment (start 110.200001 76.850001) (end 110 76.65) (width 0.4) (layer F.Cu) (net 10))
 (segment (start 110 76.65) (end 110 75.25) (width 0.4) (layer F.Cu) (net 10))
 (segment (start 116.15 76.05) (end 114.930002 76.05) (width 0.4) (layer F.Cu) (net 10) (status 30))
 (segment (start 114.95 76.15) (end 114.9 76.1) (width 0.4) (layer F.Cu) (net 10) (status 30))
 (segment (start 115.05 76.05) (end 114.95 76.15) (width 0.4) (layer F.Cu) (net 10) (status 30))
 (segment (start 116.15 76.05) (end 115.05 76.05) (width 0.4) (layer F.Cu) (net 10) (status 30))
 (segment (start 110 73.85) (end 110 75.25) (width 0.4) (layer F.Cu) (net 10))
 (segment (start 110 71.195) (end 110 73.85) (width 0.4) (layer F.Cu) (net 10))
 (segment (start 107.75 68.945) (end 110 71.195) (width 0.4) (layer F.Cu) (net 10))
 (segment (start 106.35 68.945) (end 107.75 68.945) (width 0.4) (layer F.Cu) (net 10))
 (segment (start 139 76.7) (end 139.2 76.9) (width 0.4) (layer F.Cu) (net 11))
 (segment (start 138.35 76.05) (end 139.2 76.9) (width 0.4) (layer F.Cu) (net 11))
 (segment (start 132.15 76.05) (end 138.35 76.05) (width 0.4) (layer F.Cu) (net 11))
 (segment (start 152.700001 85.000001) (end 159.299999 85.000001) (width 0.4) (layer F.Cu) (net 12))
 (segment (start 150.5 82.8) (end 152.700001 85.000001) (width 0.4) (layer F.Cu) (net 12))
 (segment (start 130.7 82.8) (end 150.5 82.8) (width 0.4) (layer F.Cu) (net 12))
 (segment (start 128.95 84.55) (end 130.7 82.8) (width 0.4) (layer F.Cu) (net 12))
 (segment (start 124.969998 84.55) (end 128.95 84.55) (width 0.4) (layer F.Cu) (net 12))
 (segment (start 124.2 83.780002) (end 124.969998 84.55) (width 0.4) (layer F.Cu) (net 12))
 (segment (start 124.2 78.1) (end 124.2 83.780002) (width 0.4) (layer F.Cu) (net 12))
 (segment (start 159.299999 85.000001) (end 161.4 85) (width 0.4) (layer F.Cu) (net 12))
 (segment (start 130.25 72.05) (end 124.2 78.1) (width 0.4) (layer F.Cu) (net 12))
 (segment (start 132.15 72.05) (end 130.25 72.05) (width 0.4) (layer F.Cu) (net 12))
 (segment (start 137 67.79) (end 137 67.82) (width 0.4) (layer F.Cu) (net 15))
 (segment (start 137 67.82) (end 134.6 67.82) (width 0.4) (layer F.Cu) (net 15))
 (segment (start 134.6 66.6) (end 134.6 67.82) (width 0.4) (layer F.Cu) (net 15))
 (segment (start 134.6 67.82) (end 134.6 72.02) (width 0.4) (layer F.Cu) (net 15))
 (segment (start 132.15 66.05) (end 134.05 66.05) (width 0.4) (layer F.Cu) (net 15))
 (segment (start 134.05 66.05) (end 134.6 66.6) (width 0.4) (layer F.Cu) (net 15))
 (segment (start 134.6 72.02) (end 135.45 72.87) (width 0.4) (layer F.Cu) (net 15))
 (segment (start 135.45 72.87) (end 141.9 72.87) (width 0.4) (layer F.Cu) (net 15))
 (segment (start 141.9 72.87) (end 141.9 69.45) (width 0.4) (layer F.Cu) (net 15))
 (segment (start 141.825001 69.524999) (end 141.9 69.45) (width 0.4) (layer F.Cu) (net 15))
 (segment (start 136.209998 67.79) (end 137 67.79) (width 0.4) (layer F.Cu) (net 15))
 (segment (start 136.6 64.85) (end 137 65.25) (width 0.4) (layer F.Cu) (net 16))
 (segment (start 134.05 64.05) (end 132.15 64.05) (width 0.4) (layer F.Cu) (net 16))
 (segment (start 134.15 64.05) (end 134.05 64.05) (width 0.4) (layer F.Cu) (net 16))
 (segment (start 135.35 65.25) (end 134.15 64.05) (width 0.4) (layer F.Cu) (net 16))
 (segment (start 137 65.25) (end 135.35 65.25) (width 0.4) (layer F.Cu) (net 16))
 (segment (start 132.15 74.05) (end 140.1 74.05) (width 0.4) (layer F.Cu) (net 17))
 (segment (start 140.1 74.05) (end 141.55 75.5) (width 0.4) (layer F.Cu) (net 17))
 (segment (start 141.55 75.5) (end 141.55 76.9) (width 0.4) (layer F.Cu) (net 17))
 (segment (start 157.7 65.5) (end 162.25 65.5) (width 0.4) (layer F.Cu) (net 18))
 (segment (start 162.25 65.5) (end 162.9 66.15) (width 0.4) (layer F.Cu) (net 18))
 (segment (start 161.1 87.2) (end 161.4 87.5) (width 0.4) (layer F.Cu) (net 19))
 (segment (start 158.2 87.1) (end 158.3 87.2) (width 0.4) (layer F.Cu) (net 19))
 (segment (start 158.6 87.5) (end 158.2 87.1) (width 0.4) (layer F.Cu) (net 19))
 (segment (start 161.4 87.5) (end 158.6 87.5) (width 0.4) (layer F.Cu) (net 19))
 (segment (start 158 83.6) (end 158.2 83.6) (width 0.4) (layer F.Cu) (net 20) (status 30))
 (segment (start 161.4 83.4) (end 161.4 82.5) (width 0.4) (layer F.Cu) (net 20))
 (segment (start 161.2 83.6) (end 161.4 83.4) (width 0.4) (layer F.Cu) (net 20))
 (segment (start 158.2 83.6) (end 161.2 83.6) (width 0.4) (layer F.Cu) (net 20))
 (segment (start 146.75 68.9) (end 151.9 68.9) (width 0.4) (layer F.Cu) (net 21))
 (segment (start 151.9 68.9) (end 152 68.8) (width 0.4) (layer F.Cu) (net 21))
 (segment (start 141.9 66.625) (end 141.9 66.15) (width 0.4) (layer F.Cu) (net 22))
 (segment (start 146.1 66.15) (end 146.75 65.5) (width 0.4) (layer F.Cu) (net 22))
 (segment (start 141.9 66.15) (end 146.1 66.15) (width 0.4) (layer F.Cu) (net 22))
 (segment (start 141.55 80.3) (end 145.25 80.3) (width 0.4) (layer F.Cu) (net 4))
 (segment (start 145.25 80.780002) (end 145.25 80.3) (width 0.4) (layer F.Cu) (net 4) (status 30))
 (segment (start 132.15 70.05) (end 133.35 70.05) (width 0.4) (layer F.Cu) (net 13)))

